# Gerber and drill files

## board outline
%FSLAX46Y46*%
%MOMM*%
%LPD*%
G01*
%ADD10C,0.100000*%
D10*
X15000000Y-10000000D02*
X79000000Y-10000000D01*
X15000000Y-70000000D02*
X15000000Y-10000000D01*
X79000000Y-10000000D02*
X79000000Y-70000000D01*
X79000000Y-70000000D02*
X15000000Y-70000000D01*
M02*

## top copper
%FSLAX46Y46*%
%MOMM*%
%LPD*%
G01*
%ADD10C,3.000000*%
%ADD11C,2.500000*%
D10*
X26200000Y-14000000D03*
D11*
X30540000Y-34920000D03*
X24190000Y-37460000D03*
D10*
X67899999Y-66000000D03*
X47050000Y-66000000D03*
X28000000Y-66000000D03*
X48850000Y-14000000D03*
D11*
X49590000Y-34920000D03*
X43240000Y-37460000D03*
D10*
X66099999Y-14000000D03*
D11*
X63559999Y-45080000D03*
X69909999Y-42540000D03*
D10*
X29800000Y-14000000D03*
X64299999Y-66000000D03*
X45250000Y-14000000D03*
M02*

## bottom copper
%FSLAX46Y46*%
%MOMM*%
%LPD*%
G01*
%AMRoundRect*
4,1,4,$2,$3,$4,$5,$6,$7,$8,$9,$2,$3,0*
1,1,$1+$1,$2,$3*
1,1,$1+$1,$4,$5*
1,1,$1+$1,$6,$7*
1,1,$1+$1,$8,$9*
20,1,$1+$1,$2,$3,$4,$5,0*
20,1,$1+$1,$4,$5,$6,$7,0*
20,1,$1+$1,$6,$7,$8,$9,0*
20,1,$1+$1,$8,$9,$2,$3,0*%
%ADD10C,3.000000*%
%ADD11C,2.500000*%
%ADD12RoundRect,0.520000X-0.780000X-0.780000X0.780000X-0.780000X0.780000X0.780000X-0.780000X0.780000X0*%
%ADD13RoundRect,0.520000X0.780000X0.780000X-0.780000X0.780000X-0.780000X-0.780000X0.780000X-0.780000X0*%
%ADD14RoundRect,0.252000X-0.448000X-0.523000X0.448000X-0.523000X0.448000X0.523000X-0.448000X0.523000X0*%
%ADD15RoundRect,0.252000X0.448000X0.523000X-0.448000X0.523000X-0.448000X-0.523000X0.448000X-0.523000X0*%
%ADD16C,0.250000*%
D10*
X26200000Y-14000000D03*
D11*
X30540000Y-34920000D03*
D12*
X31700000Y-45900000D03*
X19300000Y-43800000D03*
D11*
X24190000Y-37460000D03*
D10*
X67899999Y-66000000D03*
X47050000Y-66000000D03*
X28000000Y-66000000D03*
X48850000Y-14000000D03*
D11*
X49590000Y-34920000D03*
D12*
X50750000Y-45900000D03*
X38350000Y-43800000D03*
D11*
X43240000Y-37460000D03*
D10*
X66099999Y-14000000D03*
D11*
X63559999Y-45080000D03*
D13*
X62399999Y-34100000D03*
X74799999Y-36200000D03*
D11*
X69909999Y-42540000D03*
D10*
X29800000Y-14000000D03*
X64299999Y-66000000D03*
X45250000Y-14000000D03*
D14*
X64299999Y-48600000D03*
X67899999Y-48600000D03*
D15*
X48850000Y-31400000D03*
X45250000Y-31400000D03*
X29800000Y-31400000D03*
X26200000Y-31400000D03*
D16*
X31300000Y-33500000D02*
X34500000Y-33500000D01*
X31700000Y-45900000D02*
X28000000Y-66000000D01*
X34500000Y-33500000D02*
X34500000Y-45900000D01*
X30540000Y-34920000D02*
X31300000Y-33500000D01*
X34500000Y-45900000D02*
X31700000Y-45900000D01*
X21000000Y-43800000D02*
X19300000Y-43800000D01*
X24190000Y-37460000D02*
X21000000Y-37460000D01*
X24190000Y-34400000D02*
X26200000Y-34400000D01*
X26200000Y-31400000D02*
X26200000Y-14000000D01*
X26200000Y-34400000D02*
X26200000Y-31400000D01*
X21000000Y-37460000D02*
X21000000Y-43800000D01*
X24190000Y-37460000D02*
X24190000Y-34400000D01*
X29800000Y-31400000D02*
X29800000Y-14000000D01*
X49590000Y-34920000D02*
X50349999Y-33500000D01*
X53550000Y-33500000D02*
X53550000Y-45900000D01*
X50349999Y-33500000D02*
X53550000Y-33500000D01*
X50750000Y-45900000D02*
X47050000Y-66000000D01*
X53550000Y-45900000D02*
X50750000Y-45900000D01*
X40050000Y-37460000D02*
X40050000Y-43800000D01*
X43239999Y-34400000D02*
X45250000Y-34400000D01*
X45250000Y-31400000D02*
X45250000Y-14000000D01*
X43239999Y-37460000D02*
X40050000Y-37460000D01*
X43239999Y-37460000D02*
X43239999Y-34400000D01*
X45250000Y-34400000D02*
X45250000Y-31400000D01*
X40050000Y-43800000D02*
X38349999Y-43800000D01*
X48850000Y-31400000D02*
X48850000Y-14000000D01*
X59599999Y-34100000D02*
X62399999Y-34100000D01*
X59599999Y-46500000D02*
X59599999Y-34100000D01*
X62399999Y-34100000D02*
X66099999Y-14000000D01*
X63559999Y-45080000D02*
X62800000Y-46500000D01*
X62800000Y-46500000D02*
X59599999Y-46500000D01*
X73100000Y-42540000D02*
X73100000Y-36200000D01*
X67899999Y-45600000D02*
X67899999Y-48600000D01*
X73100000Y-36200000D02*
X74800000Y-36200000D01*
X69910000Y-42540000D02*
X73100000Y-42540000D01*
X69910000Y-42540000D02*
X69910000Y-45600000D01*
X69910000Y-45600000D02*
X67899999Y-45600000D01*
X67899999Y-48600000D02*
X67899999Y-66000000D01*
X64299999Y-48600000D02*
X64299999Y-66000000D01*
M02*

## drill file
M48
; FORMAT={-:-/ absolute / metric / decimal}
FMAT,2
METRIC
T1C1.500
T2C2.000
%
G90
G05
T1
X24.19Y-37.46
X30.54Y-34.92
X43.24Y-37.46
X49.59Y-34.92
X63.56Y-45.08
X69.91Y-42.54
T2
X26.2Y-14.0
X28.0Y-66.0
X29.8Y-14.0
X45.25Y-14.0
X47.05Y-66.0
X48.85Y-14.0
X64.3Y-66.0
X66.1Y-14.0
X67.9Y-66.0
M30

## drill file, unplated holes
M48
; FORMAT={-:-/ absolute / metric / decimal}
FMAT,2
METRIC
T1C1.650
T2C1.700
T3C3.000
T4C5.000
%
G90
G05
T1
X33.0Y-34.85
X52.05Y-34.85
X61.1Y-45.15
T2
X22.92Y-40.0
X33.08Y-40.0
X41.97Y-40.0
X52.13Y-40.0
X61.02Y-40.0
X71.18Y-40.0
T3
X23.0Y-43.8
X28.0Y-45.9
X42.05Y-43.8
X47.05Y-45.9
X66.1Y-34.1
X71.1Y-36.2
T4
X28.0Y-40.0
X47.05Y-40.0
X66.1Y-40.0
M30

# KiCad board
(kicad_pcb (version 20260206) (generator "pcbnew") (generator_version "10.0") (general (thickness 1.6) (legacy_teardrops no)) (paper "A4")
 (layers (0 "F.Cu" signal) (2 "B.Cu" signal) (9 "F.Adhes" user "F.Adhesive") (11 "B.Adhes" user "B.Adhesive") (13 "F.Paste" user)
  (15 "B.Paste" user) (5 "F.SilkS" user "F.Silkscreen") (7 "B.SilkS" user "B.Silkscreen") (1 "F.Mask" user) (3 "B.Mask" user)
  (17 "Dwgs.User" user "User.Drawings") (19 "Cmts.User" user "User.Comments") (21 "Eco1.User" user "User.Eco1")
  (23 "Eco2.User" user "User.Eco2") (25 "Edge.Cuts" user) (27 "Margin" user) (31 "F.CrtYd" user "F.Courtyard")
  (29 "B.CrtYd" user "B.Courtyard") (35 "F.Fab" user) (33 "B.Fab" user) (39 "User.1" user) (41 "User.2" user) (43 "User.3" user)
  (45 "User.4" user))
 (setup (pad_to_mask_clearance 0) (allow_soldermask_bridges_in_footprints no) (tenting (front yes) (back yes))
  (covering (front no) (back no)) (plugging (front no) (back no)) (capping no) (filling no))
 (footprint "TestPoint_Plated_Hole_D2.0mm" (layer "F.Cu") (at 26.2 14)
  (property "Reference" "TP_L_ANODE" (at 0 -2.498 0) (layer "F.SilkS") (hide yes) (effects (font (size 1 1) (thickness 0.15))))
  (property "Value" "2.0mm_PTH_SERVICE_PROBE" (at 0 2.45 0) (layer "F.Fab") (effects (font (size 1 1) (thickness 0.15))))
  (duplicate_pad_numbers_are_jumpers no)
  (pad "1" thru_hole circle (at 0 0) (size 3 3) (drill 2) (layers "*.Cu" "*.Mask") (remove_unused_layers no) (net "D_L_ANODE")))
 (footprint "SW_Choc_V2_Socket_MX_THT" (layer "F.Cu") (at 28 40)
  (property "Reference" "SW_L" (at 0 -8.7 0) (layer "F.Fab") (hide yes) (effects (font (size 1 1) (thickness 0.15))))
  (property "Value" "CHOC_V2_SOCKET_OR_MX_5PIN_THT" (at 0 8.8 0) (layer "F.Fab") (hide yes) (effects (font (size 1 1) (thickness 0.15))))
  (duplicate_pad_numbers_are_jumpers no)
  (pad "" np_thru_hole circle (at -5.08 0) (size 1.7 1.7) (drill 1.7) (layers "*.Cu" "*.Mask"))
  (pad "" np_thru_hole circle (at -5 3.8) (size 3 3) (drill 3) (layers "*.Cu" "*.Mask"))
  (pad "" np_thru_hole circle (at 0 0) (size 5 5) (drill 5) (layers "*.Cu" "*.Mask"))
  (pad "" np_thru_hole circle (at 0 5.9) (size 3 3) (drill 3) (layers "*.Cu" "*.Mask"))
  (pad "" np_thru_hole circle (at 5 -5.15) (size 1.65 1.65) (drill 1.65) (layers "*.Cu" "*.Mask"))
  (pad "" np_thru_hole circle (at 5.08 0) (size 1.7 1.7) (drill 1.7) (layers "*.Cu" "*.Mask"))
  (pad "1" thru_hole circle (at 2.54 -5.08) (size 2.5 2.5) (drill 1.5) (layers "*.Cu" "*.Mask") (remove_unused_layers no) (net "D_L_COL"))
  (pad "1" smd roundrect (at 3.7 5.9) (size 2.6 2.6) (layers "B.Cu" "B.Mask" "B.Paste") (roundrect_rratio 0.2) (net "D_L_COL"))
  (pad "2" smd roundrect (at -8.7 3.8) (size 2.6 2.6) (layers "B.Cu" "B.Mask" "B.Paste") (roundrect_rratio 0.2) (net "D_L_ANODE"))
  (pad "2" thru_hole circle (at -3.81 -2.54) (size 2.5 2.5) (drill 1.5) (layers "*.Cu" "*.Mask") (remove_unused_layers no) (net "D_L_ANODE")))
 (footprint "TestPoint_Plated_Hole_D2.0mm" (layer "F.Cu") (at 67.899999 66)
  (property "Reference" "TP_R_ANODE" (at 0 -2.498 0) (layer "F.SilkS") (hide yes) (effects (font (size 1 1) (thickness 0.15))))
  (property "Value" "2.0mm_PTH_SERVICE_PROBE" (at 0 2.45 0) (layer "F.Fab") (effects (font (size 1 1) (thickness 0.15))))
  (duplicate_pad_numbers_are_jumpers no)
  (pad "1" thru_hole circle (at 0 0) (size 3 3) (drill 2) (layers "*.Cu" "*.Mask") (remove_unused_layers no) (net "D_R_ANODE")))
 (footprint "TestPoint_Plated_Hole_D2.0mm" (layer "F.Cu") (at 47.05 66)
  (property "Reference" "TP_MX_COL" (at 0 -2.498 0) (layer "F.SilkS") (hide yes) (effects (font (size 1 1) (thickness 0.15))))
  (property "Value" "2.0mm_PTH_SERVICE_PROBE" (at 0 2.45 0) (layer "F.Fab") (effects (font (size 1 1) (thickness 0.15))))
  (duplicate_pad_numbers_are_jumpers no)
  (pad "1" thru_hole circle (at 0 0) (size 3 3) (drill 2) (layers "*.Cu" "*.Mask") (remove_unused_layers no) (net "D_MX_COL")))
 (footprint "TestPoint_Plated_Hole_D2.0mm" (layer "F.Cu") (at 28 66)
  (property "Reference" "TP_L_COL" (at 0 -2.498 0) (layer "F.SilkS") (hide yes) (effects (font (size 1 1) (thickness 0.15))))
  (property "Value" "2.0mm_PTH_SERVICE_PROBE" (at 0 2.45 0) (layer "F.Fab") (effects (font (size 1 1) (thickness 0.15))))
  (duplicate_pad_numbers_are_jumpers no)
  (pad "1" thru_hole circle (at 0 0) (size 3 3) (drill 2) (layers "*.Cu" "*.Mask") (remove_unused_layers no) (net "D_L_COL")))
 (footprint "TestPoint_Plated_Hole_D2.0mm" (layer "F.Cu") (at 48.85 14)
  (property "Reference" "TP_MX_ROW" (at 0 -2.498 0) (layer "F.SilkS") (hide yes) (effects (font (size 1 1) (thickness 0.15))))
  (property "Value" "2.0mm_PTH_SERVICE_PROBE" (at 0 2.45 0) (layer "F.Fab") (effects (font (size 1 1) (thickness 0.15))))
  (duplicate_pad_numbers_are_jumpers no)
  (pad "1" thru_hole circle (at 0 0) (size 3 3) (drill 2) (layers "*.Cu" "*.Mask") (remove_unused_layers no) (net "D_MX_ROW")))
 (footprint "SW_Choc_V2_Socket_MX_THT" (layer "F.Cu") (at 47.05 40)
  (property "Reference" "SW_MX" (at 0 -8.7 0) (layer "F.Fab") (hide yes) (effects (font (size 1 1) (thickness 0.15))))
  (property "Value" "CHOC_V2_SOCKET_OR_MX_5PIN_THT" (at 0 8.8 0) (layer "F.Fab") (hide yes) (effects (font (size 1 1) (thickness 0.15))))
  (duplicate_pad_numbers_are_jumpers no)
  (pad "" np_thru_hole circle (at -5.08 0) (size 1.7 1.7) (drill 1.7) (layers "*.Cu" "*.Mask"))
  (pad "" np_thru_hole circle (at -5 3.8) (size 3 3) (drill 3) (layers "*.Cu" "*.Mask"))
  (pad "" np_thru_hole circle (at 0 0) (size 5 5) (drill 5) (layers "*.Cu" "*.Mask"))
  (pad "" np_thru_hole circle (at 0 5.9) (size 3 3) (drill 3) (layers "*.Cu" "*.Mask"))
  (pad "" np_thru_hole circle (at 5 -5.15) (size 1.65 1.65) (drill 1.65) (layers "*.Cu" "*.Mask"))
  (pad "" np_thru_hole circle (at 5.08 0) (size 1.7 1.7) (drill 1.7) (layers "*.Cu" "*.Mask"))
  (pad "1" thru_hole circle (at 2.54 -5.08) (size 2.5 2.5) (drill 1.5) (layers "*.Cu" "*.Mask") (remove_unused_layers no) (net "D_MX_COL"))
  (pad "1" smd roundrect (at 3.7 5.9) (size 2.6 2.6) (layers "B.Cu" "B.Mask" "B.Paste") (roundrect_rratio 0.2) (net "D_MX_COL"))
  (pad "2" smd roundrect (at -8.7 3.8) (size 2.6 2.6) (layers "B.Cu" "B.Mask" "B.Paste") (roundrect_rratio 0.2) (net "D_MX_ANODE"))
  (pad "2" thru_hole circle (at -3.81 -2.54) (size 2.5 2.5) (drill 1.5) (layers "*.Cu" "*.Mask") (remove_unused_layers no)
   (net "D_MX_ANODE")))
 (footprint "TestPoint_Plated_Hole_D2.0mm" (layer "F.Cu") (at 66.099999 14)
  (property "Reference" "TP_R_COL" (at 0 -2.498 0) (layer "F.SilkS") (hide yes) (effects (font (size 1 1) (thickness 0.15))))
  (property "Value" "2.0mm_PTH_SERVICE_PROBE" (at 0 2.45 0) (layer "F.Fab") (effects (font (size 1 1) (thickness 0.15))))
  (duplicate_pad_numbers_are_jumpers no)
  (pad "1" thru_hole circle (at 0 0) (size 3 3) (drill 2) (layers "*.Cu" "*.Mask") (remove_unused_layers no) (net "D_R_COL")))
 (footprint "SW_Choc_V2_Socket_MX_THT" (layer "F.Cu") (at 66.099999 40 180)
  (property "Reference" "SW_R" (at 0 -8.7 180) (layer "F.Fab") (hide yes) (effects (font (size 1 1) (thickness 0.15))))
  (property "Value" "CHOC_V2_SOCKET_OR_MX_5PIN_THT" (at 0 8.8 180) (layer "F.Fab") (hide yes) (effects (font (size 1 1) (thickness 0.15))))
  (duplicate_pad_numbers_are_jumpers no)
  (pad "" np_thru_hole circle (at -5.08 0 180) (size 1.7 1.7) (drill 1.7) (layers "*.Cu" "*.Mask"))
  (pad "" np_thru_hole circle (at -5 3.8 180) (size 3 3) (drill 3) (layers "*.Cu" "*.Mask"))
  (pad "" np_thru_hole circle (at 0 0 180) (size 5 5) (drill 5) (layers "*.Cu" "*.Mask"))
  (pad "" np_thru_hole circle (at 0 5.9 180) (size 3 3) (drill 3) (layers "*.Cu" "*.Mask"))
  (pad "" np_thru_hole circle (at 5 -5.15 180) (size 1.65 1.65) (drill 1.65) (layers "*.Cu" "*.Mask"))
  (pad "" np_thru_hole circle (at 5.08 0 180) (size 1.7 1.7) (drill 1.7) (layers "*.Cu" "*.Mask"))
  (pad "1" thru_hole circle (at 2.54 -5.08 180) (size 2.5 2.5) (drill 1.5) (layers "*.Cu" "*.Mask") (remove_unused_layers no)
   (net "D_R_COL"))
  (pad "1" smd roundrect (at 3.7 5.9 180) (size 2.6 2.6) (layers "B.Cu" "B.Mask" "B.Paste") (roundrect_rratio 0.2) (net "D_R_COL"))
  (pad "2" smd roundrect (at -8.7 3.8 180) (size 2.6 2.6) (layers "B.Cu" "B.Mask" "B.Paste") (roundrect_rratio 0.2) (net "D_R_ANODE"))
  (pad "2" thru_hole circle (at -3.81 -2.54 180) (size 2.5 2.5) (drill 1.5) (layers "*.Cu" "*.Mask") (remove_unused_layers no)
   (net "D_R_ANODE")))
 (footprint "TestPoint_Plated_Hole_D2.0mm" (layer "F.Cu") (at 29.8 14)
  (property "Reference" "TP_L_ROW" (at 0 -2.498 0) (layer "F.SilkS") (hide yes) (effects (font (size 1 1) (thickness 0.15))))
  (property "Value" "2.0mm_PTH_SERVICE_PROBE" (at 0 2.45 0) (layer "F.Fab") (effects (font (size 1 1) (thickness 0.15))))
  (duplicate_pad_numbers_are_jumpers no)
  (pad "1" thru_hole circle (at 0 0) (size 3 3) (drill 2) (layers "*.Cu" "*.Mask") (remove_unused_layers no) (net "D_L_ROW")))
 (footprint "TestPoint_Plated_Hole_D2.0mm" (layer "F.Cu") (at 64.299999 66)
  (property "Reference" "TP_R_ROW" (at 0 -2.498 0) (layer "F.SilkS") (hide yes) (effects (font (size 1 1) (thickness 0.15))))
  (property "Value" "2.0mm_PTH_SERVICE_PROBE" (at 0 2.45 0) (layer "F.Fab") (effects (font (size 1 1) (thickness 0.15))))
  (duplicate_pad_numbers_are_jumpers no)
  (pad "1" thru_hole circle (at 0 0) (size 3 3) (drill 2) (layers "*.Cu" "*.Mask") (remove_unused_layers no) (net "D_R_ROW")))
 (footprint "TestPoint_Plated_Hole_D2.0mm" (layer "F.Cu") (at 45.25 14)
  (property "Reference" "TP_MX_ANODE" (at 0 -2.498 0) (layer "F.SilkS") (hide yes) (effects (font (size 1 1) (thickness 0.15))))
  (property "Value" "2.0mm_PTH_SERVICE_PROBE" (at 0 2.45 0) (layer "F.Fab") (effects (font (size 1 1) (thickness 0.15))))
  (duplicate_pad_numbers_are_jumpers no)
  (pad "1" thru_hole circle (at 0 0) (size 3 3) (drill 2) (layers "*.Cu" "*.Mask") (remove_unused_layers no) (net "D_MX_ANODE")))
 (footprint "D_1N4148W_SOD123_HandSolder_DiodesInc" (layer "B.Cu") (at 66.099999 48.6)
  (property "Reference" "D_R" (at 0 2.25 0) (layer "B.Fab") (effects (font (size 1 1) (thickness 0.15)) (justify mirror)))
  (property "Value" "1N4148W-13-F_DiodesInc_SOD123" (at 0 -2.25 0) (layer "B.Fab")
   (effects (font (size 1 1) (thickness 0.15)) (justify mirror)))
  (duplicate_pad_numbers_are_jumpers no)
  (pad "1" smd roundrect (at -1.8 0) (size 1.4 1.55) (layers "B.Cu" "B.Mask" "B.Paste") (roundrect_rratio 0.18) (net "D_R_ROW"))
  (pad "2" smd roundrect (at 1.8 0) (size 1.4 1.55) (layers "B.Cu" "B.Mask" "B.Paste") (roundrect_rratio 0.18) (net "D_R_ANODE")))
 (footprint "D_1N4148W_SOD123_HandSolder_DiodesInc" (layer "B.Cu") (at 47.05 31.4 180)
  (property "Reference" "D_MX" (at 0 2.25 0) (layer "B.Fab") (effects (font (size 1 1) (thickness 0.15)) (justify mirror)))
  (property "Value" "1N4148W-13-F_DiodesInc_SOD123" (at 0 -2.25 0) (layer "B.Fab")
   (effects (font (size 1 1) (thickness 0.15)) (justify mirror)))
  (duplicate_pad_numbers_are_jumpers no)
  (pad "1" smd roundrect (at -1.8 0 180) (size 1.4 1.55) (layers "B.Cu" "B.Mask" "B.Paste") (roundrect_rratio 0.18) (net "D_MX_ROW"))
  (pad "2" smd roundrect (at 1.8 0 180) (size 1.4 1.55) (layers "B.Cu" "B.Mask" "B.Paste") (roundrect_rratio 0.18) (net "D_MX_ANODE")))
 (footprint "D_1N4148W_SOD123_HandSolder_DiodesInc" (layer "B.Cu") (at 28 31.4 180)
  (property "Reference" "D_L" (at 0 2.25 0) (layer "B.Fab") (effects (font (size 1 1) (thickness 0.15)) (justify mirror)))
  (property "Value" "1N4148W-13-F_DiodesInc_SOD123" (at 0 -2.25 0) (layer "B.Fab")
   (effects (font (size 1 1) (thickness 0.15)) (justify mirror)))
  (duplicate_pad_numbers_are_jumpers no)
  (pad "1" smd roundrect (at -1.8 0 180) (size 1.4 1.55) (layers "B.Cu" "B.Mask" "B.Paste") (roundrect_rratio 0.18) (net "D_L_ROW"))
  (pad "2" smd roundrect (at 1.8 0 180) (size 1.4 1.55) (layers "B.Cu" "B.Mask" "B.Paste") (roundrect_rratio 0.18) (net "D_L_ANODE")))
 (gr_line (start 15 10) (end 79 10) (stroke (width 0.1) (type default)) (layer "Edge.Cuts"))
 (gr_line (start 15 70) (end 15 10) (stroke (width 0.1) (type default)) (layer "Edge.Cuts"))
 (gr_line (start 79 10) (end 79 70) (stroke (width 0.1) (type default)) (layer "Edge.Cuts"))
 (gr_line (start 79 70) (end 15 70) (stroke (width 0.1) (type default)) (layer "Edge.Cuts"))
 (segment (start 31.3 33.5) (end 34.5 33.5) (width 0.25) (layer "B.Cu") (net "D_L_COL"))
 (segment (start 31.7 45.9) (end 28 66) (width 0.25) (layer "B.Cu") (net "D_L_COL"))
 (segment (start 34.5 33.5) (end 34.5 45.9) (width 0.25) (layer "B.Cu") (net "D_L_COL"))
 (segment (start 30.54 34.92) (end 31.3 33.5) (width 0.25) (layer "B.Cu") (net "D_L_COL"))
 (segment (start 34.5 45.9) (end 31.7 45.9) (width 0.25) (layer "B.Cu") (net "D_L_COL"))
 (segment (start 21 43.8) (end 19.3 43.8) (width 0.25) (layer "B.Cu") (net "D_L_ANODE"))
 (segment (start 24.19 37.46) (end 21 37.46) (width 0.25) (layer "B.Cu") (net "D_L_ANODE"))
 (segment (start 24.19 34.4) (end 26.2 34.4) (width 0.25) (layer "B.Cu") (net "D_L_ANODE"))
 (segment (start 26.2 31.4) (end 26.2 14) (width 0.25) (layer "B.Cu") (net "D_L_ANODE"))
 (segment (start 26.2 34.4) (end 26.2 31.4) (width 0.25) (layer "B.Cu") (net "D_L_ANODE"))
 (segment (start 21 37.46) (end 21 43.8) (width 0.25) (layer "B.Cu") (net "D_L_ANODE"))
 (segment (start 24.19 37.46) (end 24.19 34.4) (width 0.25) (layer "B.Cu") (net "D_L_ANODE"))
 (segment (start 29.8 31.4) (end 29.8 14) (width 0.25) (layer "B.Cu") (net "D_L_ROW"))
 (segment (start 49.59 34.92) (end 50.349999 33.5) (width 0.25) (layer "B.Cu") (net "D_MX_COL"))
 (segment (start 53.55 33.5) (end 53.55 45.9) (width 0.25) (layer "B.Cu") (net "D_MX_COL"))
 (segment (start 50.349999 33.5) (end 53.55 33.5) (width 0.25) (layer "B.Cu") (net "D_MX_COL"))
 (segment (start 50.75 45.9) (end 47.05 66) (width 0.25) (layer "B.Cu") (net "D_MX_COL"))
 (segment (start 53.55 45.9) (end 50.75 45.9) (width 0.25) (layer "B.Cu") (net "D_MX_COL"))
 (segment (start 40.05 37.46) (end 40.05 43.8) (width 0.25) (layer "B.Cu") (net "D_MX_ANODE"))
 (segment (start 43.239999 34.4) (end 45.25 34.4) (width 0.25) (layer "B.Cu") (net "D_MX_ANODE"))
 (segment (start 45.25 31.4) (end 45.25 14) (width 0.25) (layer "B.Cu") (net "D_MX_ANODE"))
 (segment (start 43.239999 37.46) (end 40.05 37.46) (width 0.25) (layer "B.Cu") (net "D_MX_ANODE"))
 (segment (start 43.239999 37.46) (end 43.239999 34.4) (width 0.25) (layer "B.Cu") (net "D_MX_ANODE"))
 (segment (start 45.25 34.4) (end 45.25 31.4) (width 0.25) (layer "B.Cu") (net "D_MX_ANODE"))
 (segment (start 40.05 43.8) (end 38.349999 43.8) (width 0.25) (layer "B.Cu") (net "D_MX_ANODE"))
 (segment (start 48.85 31.4) (end 48.85 14) (width 0.25) (layer "B.Cu") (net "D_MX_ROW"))
 (segment (start 59.599999 34.1) (end 62.399999 34.1) (width 0.25) (layer "B.Cu") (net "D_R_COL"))
 (segment (start 59.599999 46.5) (end 59.599999 34.1) (width 0.25) (layer "B.Cu") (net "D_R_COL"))
 (segment (start 62.399999 34.1) (end 66.099999 14) (width 0.25) (layer "B.Cu") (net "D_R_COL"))
 (segment (start 63.559999 45.08) (end 62.8 46.5) (width 0.25) (layer "B.Cu") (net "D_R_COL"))
 (segment (start 62.8 46.5) (end 59.599999 46.5) (width 0.25) (layer "B.Cu") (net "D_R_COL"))
 (segment (start 73.1 42.54) (end 73.1 36.2) (width 0.25) (layer "B.Cu") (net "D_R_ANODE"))
 (segment (start 67.899999 45.6) (end 67.899999 48.6) (width 0.25) (layer "B.Cu") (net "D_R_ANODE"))
 (segment (start 73.1 36.2) (end 74.8 36.2) (width 0.25) (layer "B.Cu") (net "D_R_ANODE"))
 (segment (start 69.91 42.54) (end 73.1 42.54) (width 0.25) (layer "B.Cu") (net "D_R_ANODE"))
 (segment (start 69.91 42.54) (end 69.91 45.6) (width 0.25) (layer "B.Cu") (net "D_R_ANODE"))
 (segment (start 69.91 45.6) (end 67.899999 45.6) (width 0.25) (layer "B.Cu") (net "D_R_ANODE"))
 (segment (start 67.899999 48.6) (end 67.899999 66) (width 0.25) (layer "B.Cu") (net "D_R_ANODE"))
 (segment (start 64.299999 48.6) (end 64.299999 66) (width 0.25) (layer "B.Cu") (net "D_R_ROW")))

